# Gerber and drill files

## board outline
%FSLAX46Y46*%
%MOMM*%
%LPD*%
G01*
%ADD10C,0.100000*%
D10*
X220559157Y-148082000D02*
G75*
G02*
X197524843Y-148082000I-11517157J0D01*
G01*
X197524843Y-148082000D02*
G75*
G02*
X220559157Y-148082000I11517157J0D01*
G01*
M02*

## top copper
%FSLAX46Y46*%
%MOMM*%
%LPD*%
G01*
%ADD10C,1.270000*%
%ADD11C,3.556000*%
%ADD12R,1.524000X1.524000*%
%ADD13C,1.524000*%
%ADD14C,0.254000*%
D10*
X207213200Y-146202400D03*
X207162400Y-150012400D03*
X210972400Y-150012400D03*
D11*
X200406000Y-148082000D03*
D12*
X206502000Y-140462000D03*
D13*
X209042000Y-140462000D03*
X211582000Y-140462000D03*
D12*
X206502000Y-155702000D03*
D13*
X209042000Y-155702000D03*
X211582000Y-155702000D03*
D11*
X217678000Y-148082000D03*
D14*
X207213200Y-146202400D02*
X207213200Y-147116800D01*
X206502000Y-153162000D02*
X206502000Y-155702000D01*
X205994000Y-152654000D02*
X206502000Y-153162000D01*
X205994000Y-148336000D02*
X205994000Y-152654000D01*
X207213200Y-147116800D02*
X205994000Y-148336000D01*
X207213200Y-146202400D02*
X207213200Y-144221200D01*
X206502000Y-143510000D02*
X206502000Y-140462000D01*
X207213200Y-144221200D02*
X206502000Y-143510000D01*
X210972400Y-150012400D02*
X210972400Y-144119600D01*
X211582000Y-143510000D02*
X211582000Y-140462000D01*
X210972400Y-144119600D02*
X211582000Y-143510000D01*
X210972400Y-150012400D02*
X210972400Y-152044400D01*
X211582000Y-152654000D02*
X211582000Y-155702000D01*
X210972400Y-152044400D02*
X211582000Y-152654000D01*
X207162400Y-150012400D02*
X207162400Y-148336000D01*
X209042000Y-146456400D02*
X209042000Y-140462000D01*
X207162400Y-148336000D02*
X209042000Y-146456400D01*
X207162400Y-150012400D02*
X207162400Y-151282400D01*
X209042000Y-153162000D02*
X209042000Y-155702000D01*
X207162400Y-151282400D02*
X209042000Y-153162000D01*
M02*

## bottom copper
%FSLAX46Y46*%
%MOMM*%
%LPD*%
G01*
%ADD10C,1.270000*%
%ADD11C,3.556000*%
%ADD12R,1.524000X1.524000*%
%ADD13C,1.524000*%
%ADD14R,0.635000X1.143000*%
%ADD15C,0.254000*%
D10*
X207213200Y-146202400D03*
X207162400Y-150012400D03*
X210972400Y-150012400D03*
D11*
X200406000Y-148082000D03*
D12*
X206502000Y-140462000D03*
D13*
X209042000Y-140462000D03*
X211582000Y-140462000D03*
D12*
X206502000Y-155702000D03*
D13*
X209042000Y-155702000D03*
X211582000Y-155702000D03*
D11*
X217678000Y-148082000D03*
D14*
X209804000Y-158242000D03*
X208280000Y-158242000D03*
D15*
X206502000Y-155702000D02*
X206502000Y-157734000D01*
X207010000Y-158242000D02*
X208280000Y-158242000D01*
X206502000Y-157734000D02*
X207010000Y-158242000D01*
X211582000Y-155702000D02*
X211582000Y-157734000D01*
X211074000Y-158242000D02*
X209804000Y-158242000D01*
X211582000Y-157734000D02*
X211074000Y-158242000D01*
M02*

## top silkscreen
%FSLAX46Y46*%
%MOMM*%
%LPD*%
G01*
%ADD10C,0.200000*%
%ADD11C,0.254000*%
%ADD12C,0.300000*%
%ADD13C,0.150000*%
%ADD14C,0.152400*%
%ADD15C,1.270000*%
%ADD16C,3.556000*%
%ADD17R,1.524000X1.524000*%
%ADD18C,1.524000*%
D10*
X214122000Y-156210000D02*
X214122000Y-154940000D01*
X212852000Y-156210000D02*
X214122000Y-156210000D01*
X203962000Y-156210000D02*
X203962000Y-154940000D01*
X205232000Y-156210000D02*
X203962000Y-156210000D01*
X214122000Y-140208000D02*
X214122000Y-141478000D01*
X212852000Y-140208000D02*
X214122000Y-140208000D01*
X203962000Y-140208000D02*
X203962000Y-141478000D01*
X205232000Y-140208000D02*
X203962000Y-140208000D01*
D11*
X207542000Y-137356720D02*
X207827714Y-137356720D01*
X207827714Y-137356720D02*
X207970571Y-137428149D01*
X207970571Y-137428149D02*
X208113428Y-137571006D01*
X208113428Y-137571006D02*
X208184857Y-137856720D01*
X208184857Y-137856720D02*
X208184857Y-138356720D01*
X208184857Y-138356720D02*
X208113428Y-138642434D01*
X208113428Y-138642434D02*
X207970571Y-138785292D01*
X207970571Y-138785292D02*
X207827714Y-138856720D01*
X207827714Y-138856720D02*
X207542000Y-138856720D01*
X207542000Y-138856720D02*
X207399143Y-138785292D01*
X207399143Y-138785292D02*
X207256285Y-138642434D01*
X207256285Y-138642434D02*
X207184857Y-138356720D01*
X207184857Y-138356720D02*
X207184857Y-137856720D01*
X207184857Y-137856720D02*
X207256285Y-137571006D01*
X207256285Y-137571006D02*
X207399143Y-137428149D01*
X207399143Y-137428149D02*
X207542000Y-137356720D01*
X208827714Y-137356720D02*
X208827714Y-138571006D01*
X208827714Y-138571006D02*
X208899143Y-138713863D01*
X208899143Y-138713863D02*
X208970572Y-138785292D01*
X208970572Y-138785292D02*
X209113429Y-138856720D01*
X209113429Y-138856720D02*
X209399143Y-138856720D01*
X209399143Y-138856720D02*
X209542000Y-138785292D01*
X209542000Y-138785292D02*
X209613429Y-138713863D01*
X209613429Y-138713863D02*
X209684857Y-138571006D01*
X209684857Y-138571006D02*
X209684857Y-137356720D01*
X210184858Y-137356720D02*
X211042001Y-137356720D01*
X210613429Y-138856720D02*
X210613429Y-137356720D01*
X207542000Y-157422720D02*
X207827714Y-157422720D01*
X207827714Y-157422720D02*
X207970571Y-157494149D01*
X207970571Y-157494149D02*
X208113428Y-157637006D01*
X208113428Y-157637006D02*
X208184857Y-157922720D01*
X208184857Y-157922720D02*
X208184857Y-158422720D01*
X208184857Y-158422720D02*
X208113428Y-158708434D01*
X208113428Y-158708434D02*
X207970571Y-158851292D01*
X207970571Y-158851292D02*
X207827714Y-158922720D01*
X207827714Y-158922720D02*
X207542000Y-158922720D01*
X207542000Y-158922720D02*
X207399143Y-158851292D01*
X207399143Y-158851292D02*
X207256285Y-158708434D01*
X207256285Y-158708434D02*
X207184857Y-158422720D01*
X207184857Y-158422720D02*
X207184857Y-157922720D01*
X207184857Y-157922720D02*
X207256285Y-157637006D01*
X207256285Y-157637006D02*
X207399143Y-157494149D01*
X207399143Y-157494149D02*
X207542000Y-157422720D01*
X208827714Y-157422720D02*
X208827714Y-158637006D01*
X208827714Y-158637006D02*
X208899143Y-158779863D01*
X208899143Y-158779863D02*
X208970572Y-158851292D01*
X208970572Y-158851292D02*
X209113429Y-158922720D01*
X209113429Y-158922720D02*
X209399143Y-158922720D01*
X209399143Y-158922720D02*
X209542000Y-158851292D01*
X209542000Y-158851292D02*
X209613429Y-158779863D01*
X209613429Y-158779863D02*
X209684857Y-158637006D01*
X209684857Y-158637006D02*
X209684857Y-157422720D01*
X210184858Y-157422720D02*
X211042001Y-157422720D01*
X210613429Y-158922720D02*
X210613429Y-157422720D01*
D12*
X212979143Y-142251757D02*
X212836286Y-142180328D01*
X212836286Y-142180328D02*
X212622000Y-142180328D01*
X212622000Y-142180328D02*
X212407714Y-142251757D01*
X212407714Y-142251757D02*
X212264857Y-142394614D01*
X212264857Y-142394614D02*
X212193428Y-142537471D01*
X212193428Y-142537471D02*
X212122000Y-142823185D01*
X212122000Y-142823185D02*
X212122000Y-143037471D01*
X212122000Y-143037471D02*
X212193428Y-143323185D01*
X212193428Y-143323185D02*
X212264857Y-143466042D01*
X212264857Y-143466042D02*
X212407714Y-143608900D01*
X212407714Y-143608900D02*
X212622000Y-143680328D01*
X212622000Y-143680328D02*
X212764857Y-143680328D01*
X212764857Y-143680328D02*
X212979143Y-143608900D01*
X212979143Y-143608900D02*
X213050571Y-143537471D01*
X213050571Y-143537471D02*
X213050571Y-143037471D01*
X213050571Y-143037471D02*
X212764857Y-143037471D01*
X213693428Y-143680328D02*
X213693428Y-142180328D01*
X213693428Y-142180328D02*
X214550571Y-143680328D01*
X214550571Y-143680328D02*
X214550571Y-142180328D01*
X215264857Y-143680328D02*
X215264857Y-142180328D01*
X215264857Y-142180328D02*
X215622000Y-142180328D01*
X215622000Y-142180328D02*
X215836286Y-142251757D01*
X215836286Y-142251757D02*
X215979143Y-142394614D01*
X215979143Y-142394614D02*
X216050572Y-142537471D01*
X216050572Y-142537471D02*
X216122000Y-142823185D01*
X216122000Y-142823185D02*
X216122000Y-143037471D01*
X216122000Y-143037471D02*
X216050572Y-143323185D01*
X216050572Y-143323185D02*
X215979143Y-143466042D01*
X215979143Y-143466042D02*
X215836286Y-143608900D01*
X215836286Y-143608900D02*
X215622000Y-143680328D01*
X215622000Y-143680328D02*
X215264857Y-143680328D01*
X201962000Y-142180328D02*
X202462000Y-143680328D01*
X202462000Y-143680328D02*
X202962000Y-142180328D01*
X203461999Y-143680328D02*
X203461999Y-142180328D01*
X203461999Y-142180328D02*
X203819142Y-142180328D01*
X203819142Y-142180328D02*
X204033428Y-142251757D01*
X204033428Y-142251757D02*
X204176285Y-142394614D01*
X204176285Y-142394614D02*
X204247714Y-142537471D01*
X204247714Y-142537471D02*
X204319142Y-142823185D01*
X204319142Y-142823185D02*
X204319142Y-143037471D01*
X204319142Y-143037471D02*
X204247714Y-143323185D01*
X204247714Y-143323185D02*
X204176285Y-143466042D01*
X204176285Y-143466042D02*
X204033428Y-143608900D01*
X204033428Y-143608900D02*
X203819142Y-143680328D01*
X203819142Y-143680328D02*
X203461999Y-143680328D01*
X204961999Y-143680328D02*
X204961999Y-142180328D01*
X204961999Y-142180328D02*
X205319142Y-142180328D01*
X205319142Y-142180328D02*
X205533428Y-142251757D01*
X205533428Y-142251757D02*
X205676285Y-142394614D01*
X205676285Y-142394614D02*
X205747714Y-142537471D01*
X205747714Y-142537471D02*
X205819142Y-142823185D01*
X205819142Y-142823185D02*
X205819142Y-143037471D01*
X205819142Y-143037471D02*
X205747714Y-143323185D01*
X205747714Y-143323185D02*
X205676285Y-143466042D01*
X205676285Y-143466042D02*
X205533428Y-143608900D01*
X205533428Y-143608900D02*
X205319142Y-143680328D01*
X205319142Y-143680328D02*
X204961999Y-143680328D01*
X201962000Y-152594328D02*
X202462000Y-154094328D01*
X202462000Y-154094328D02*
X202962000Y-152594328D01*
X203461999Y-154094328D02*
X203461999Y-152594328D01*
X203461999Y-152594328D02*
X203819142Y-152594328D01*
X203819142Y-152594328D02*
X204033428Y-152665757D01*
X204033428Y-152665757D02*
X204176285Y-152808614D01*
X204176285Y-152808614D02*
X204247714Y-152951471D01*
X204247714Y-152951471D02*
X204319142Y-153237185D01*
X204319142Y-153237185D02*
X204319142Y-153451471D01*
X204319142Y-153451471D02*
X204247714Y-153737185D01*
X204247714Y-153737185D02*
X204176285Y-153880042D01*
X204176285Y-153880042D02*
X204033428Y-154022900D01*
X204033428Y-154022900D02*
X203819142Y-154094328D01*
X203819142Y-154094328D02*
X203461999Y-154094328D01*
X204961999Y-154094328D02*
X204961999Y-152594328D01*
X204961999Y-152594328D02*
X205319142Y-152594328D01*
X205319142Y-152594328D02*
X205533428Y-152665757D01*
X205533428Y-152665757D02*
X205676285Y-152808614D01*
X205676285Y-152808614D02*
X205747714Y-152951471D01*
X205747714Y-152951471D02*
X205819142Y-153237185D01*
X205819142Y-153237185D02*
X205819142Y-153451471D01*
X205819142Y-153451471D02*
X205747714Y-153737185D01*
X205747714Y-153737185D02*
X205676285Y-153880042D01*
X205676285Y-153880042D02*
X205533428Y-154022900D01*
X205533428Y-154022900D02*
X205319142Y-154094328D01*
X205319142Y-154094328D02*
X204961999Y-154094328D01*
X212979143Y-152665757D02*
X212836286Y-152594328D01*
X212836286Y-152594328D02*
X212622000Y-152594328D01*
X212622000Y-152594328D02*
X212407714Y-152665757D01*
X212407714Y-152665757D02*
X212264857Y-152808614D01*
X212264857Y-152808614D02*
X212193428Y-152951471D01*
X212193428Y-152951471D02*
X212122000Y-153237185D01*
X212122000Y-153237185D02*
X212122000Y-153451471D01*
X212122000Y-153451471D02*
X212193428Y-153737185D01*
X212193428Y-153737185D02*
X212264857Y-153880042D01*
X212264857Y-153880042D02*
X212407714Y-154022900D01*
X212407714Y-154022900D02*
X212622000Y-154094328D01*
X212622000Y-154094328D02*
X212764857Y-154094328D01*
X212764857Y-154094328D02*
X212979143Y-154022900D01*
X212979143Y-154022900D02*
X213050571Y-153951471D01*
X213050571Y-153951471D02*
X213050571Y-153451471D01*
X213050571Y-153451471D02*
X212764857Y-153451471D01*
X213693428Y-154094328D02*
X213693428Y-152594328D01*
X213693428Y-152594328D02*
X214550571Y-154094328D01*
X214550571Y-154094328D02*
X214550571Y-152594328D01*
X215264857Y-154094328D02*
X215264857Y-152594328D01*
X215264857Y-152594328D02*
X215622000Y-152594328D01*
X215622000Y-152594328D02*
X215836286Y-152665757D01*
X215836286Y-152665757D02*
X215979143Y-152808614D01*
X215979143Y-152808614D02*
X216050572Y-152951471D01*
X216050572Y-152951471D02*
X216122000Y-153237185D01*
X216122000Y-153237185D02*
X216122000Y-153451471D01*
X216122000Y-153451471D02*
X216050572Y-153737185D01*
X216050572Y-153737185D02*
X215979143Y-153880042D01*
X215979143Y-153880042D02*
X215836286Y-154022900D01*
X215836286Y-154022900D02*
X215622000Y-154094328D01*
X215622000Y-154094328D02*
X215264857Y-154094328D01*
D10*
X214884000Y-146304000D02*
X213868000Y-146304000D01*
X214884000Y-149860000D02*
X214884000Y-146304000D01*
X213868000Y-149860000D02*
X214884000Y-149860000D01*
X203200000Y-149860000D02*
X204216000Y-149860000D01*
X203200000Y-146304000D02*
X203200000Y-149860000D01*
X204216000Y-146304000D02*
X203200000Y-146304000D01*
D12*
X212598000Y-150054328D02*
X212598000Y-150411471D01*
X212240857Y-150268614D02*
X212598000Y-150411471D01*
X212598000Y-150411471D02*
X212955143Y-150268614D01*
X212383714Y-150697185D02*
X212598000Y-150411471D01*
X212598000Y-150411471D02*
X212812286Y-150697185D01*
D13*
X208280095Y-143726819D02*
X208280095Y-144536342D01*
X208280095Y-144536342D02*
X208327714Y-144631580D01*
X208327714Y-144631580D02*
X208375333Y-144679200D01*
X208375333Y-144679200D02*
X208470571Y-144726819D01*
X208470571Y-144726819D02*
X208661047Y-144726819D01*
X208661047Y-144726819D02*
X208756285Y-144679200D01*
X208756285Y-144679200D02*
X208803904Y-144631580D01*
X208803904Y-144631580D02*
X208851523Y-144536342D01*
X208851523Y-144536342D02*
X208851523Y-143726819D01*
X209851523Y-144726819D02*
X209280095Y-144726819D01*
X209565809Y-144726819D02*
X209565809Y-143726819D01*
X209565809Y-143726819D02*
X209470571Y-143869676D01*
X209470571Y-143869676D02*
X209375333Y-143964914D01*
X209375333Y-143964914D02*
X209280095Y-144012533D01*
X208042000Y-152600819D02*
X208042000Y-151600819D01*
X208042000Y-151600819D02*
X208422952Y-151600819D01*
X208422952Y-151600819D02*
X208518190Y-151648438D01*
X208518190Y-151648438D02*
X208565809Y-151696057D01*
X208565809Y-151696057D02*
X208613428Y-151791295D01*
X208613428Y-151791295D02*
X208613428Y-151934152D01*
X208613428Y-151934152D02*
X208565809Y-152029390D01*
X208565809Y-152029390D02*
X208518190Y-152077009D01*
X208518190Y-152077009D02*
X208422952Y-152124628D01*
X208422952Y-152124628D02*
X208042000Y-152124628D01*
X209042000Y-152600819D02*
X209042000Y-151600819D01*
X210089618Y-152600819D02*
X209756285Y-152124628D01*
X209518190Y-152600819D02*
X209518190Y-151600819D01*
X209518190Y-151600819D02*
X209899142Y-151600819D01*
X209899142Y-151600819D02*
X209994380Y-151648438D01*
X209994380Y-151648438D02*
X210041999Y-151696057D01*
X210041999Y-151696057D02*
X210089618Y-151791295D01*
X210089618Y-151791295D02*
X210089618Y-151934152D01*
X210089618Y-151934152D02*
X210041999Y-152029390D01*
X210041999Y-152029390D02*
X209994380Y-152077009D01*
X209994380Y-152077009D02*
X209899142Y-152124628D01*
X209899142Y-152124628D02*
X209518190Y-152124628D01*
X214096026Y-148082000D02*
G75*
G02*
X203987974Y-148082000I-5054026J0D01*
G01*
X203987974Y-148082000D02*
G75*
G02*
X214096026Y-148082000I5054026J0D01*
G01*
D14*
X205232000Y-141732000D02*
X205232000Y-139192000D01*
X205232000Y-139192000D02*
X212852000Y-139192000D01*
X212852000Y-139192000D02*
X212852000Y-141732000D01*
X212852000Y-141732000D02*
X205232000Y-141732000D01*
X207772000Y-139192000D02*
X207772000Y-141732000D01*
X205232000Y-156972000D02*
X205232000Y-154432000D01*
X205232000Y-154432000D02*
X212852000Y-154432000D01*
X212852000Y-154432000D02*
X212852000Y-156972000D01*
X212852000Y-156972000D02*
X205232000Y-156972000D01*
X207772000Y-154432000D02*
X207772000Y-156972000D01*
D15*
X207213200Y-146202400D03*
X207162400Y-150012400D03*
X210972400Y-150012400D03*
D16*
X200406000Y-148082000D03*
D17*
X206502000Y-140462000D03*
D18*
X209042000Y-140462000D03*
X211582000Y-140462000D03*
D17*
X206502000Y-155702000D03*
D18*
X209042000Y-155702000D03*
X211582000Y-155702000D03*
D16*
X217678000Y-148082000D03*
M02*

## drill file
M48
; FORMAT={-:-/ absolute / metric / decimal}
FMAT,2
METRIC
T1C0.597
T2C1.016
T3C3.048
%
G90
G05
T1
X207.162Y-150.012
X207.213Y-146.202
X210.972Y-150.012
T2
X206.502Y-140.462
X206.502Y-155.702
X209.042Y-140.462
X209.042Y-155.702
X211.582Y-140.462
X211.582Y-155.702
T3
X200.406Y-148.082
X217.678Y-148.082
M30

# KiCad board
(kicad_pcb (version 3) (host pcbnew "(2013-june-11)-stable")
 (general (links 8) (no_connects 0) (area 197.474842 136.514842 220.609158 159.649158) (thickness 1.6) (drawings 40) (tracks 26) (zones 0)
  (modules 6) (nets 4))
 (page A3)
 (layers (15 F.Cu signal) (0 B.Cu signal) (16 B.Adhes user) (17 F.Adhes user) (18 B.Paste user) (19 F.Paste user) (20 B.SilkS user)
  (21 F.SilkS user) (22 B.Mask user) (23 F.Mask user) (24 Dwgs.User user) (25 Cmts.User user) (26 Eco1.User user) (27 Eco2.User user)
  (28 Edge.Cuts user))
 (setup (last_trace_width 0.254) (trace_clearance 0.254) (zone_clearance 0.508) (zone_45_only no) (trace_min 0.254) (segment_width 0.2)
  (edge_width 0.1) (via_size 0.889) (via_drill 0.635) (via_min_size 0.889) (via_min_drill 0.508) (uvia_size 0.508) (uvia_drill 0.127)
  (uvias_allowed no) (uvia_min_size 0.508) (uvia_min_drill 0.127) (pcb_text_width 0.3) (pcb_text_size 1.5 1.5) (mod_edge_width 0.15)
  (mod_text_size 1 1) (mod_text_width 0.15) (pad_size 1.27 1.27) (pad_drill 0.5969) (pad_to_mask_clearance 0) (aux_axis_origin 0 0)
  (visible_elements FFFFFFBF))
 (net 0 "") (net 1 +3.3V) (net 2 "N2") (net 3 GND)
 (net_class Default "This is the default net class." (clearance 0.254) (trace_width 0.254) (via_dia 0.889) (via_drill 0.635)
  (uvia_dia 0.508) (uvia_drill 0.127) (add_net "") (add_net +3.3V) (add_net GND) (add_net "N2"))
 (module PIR (layer F.Cu) (at 209.042 148.082)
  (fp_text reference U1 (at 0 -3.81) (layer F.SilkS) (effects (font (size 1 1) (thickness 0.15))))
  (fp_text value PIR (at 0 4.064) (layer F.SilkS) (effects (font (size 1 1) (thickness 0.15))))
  (fp_circle (center 0 0) (end -3.9116 3.2004) (layer F.SilkS) (width 0.15))
  (pad 1 thru_hole circle (at -1.8288 -1.8796 180) (size 1.27 1.27) (drill 0.5969) (layers *.Cu *.Mask F.SilkS) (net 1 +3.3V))
  (pad 2 thru_hole circle (at -1.8796 1.9304 180) (size 1.27 1.27) (drill 0.5969) (layers *.Cu *.Mask F.SilkS) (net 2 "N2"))
  (pad 3 thru_hole circle (at 1.9304 1.9304 180) (size 1.27 1.27) (drill 0.5969) (layers *.Cu *.Mask F.SilkS) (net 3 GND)))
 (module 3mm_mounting (layer F.Cu) (at 200.406 148.082)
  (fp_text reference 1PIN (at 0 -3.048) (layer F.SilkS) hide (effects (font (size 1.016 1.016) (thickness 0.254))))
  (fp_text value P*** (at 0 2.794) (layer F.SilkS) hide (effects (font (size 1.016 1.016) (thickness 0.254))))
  (pad "" thru_hole circle (at 0 0) (size 3.556 3.556) (drill 3.048) (layers *.Cu *.Mask F.SilkS)))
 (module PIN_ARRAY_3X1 (layer F.Cu) (at 209.042 140.462)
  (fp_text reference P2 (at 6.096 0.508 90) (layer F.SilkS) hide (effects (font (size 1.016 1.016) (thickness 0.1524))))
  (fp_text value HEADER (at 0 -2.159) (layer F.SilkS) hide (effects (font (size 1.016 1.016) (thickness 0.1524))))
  (fp_line (start -3.81 1.27) (end -3.81 -1.27) (layer F.SilkS) (width 0.1524))
  (fp_line (start -3.81 -1.27) (end 3.81 -1.27) (layer F.SilkS) (width 0.1524))
  (fp_line (start 3.81 -1.27) (end 3.81 1.27) (layer F.SilkS) (width 0.1524))
  (fp_line (start 3.81 1.27) (end -3.81 1.27) (layer F.SilkS) (width 0.1524))
  (fp_line (start -1.27 -1.27) (end -1.27 1.27) (layer F.SilkS) (width 0.1524))
  (pad 1 thru_hole rect (at -2.54 0) (size 1.524 1.524) (drill 1.016) (layers *.Cu *.Mask F.SilkS) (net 1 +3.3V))
  (pad 2 thru_hole circle (at 0 0) (size 1.524 1.524) (drill 1.016) (layers *.Cu *.Mask F.SilkS) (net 2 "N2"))
  (pad 3 thru_hole circle (at 2.54 0) (size 1.524 1.524) (drill 1.016) (layers *.Cu *.Mask F.SilkS) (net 3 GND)))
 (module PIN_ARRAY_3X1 (layer F.Cu) (at 209.042 155.702)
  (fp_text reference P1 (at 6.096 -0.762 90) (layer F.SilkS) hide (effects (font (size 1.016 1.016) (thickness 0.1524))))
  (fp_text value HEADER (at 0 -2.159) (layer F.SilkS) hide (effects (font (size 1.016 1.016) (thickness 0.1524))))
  (fp_line (start -3.81 1.27) (end -3.81 -1.27) (layer F.SilkS) (width 0.1524))
  (fp_line (start -3.81 -1.27) (end 3.81 -1.27) (layer F.SilkS) (width 0.1524))
  (fp_line (start 3.81 -1.27) (end 3.81 1.27) (layer F.SilkS) (width 0.1524))
  (fp_line (start 3.81 1.27) (end -3.81 1.27) (layer F.SilkS) (width 0.1524))
  (fp_line (start -1.27 -1.27) (end -1.27 1.27) (layer F.SilkS) (width 0.1524))
  (pad 1 thru_hole rect (at -2.54 0) (size 1.524 1.524) (drill 1.016) (layers *.Cu *.Mask F.SilkS) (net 1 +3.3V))
  (pad 2 thru_hole circle (at 0 0) (size 1.524 1.524) (drill 1.016) (layers *.Cu *.Mask F.SilkS) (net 2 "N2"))
  (pad 3 thru_hole circle (at 2.54 0) (size 1.524 1.524) (drill 1.016) (layers *.Cu *.Mask F.SilkS) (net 3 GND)))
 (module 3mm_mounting (layer F.Cu) (at 217.678 148.082)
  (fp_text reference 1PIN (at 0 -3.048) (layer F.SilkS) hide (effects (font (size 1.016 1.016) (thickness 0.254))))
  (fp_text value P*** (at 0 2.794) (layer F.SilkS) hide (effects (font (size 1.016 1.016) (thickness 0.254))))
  (pad "" thru_hole circle (at 0 0) (size 3.556 3.556) (drill 3.048) (layers *.Cu *.Mask F.SilkS)))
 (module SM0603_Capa (layer B.Cu) (at 209.042 158.242 180)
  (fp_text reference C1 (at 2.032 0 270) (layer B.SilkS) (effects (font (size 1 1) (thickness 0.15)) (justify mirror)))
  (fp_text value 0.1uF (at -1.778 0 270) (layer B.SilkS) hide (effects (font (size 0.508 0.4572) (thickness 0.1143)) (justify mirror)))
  (pad 1 smd rect (at -0.762 0 180) (size 0.635 1.143) (layers B.Cu B.Paste B.Mask) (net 3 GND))
  (pad 2 smd rect (at 0.762 0 180) (size 0.635 1.143) (layers B.Cu B.Paste B.Mask) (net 1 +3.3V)))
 (gr_line (start 214.122 156.21) (end 214.122 154.94) (angle 90) (layer F.SilkS) (width 0.2))
 (gr_line (start 212.852 156.21) (end 214.122 156.21) (angle 90) (layer F.SilkS) (width 0.2))
 (gr_line (start 203.962 156.21) (end 203.962 154.94) (angle 90) (layer F.SilkS) (width 0.2))
 (gr_line (start 205.232 156.21) (end 203.962 156.21) (angle 90) (layer F.SilkS) (width 0.2))
 (gr_line (start 214.122 140.208) (end 214.122 141.478) (angle 90) (layer F.SilkS) (width 0.2))
 (gr_line (start 212.852 140.208) (end 214.122 140.208) (angle 90) (layer F.SilkS) (width 0.2))
 (gr_line (start 203.962 140.208) (end 203.962 141.478) (angle 90) (layer F.SilkS) (width 0.2))
 (gr_line (start 205.232 140.208) (end 203.962 140.208) (angle 90) (layer F.SilkS) (width 0.2))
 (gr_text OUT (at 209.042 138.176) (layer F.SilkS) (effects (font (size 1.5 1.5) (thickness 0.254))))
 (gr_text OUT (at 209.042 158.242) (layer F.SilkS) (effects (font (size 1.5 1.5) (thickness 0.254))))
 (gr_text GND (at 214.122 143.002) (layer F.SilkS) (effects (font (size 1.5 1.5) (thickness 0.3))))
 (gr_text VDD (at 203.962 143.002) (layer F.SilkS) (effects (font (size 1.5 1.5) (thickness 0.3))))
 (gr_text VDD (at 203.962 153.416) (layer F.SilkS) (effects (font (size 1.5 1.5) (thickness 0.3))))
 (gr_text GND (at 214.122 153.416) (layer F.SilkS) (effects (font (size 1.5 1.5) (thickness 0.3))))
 (gr_line (start 214.884 146.304) (end 213.868 146.304) (angle 90) (layer F.SilkS) (width 0.2))
 (gr_line (start 214.884 149.86) (end 214.884 146.304) (angle 90) (layer F.SilkS) (width 0.2))
 (gr_line (start 213.868 149.86) (end 214.884 149.86) (angle 90) (layer F.SilkS) (width 0.2))
 (gr_line (start 203.2 149.86) (end 204.216 149.86) (angle 90) (layer F.SilkS) (width 0.2))
 (gr_line (start 203.2 146.304) (end 203.2 149.86) (angle 90) (layer F.SilkS) (width 0.2))
 (gr_line (start 204.216 146.304) (end 203.2 146.304) (angle 90) (layer F.SilkS) (width 0.2))
 (gr_circle (center 209.042 148.082) (end 216.662 156.718) (layer Edge.Cuts) (width 0.1))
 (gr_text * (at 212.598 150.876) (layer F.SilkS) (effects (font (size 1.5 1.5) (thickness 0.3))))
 (segment (start 206.502 155.702) (end 206.502 157.734) (width 0.254) (layer B.Cu) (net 1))
 (segment (start 207.01 158.242) (end 208.28 158.242) (width 0.254) (layer B.Cu) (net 1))
 (segment (start 206.502 157.734) (end 207.01 158.242) (width 0.254) (layer B.Cu) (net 1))
 (segment (start 207.2132 146.2024) (end 207.2132 147.1168) (width 0.254) (layer F.Cu) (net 1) (status 10))
 (segment (start 206.502 153.162) (end 206.502 155.702) (width 0.254) (layer F.Cu) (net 1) (status 20))
 (segment (start 205.994 152.654) (end 206.502 153.162) (width 0.254) (layer F.Cu) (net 1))
 (segment (start 205.994 148.336) (end 205.994 152.654) (width 0.254) (layer F.Cu) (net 1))
 (segment (start 207.2132 147.1168) (end 205.994 148.336) (width 0.254) (layer F.Cu) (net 1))
 (segment (start 207.2132 146.2024) (end 207.2132 144.2212) (width 0.254) (layer F.Cu) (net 1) (status 10))
 (segment (start 206.502 143.51) (end 206.502 140.462) (width 0.254) (layer F.Cu) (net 1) (status 20))
 (segment (start 207.2132 144.2212) (end 206.502 143.51) (width 0.254) (layer F.Cu) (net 1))
 (segment (start 211.582 155.702) (end 211.582 157.734) (width 0.254) (layer B.Cu) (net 3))
 (segment (start 211.074 158.242) (end 209.804 158.242) (width 0.254) (layer B.Cu) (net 3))
 (segment (start 211.582 157.734) (end 211.074 158.242) (width 0.254) (layer B.Cu) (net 3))
 (segment (start 210.9724 150.0124) (end 210.9724 144.1196) (width 0.254) (layer F.Cu) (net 3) (status 10))
 (segment (start 211.582 143.51) (end 211.582 140.462) (width 0.254) (layer F.Cu) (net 3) (status 20))
 (segment (start 210.9724 144.1196) (end 211.582 143.51) (width 0.254) (layer F.Cu) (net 3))
 (segment (start 210.9724 150.0124) (end 210.9724 152.0444) (width 0.254) (layer F.Cu) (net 3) (status 10))
 (segment (start 211.582 152.654) (end 211.582 155.702) (width 0.254) (layer F.Cu) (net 3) (status 20))
 (segment (start 210.9724 152.0444) (end 211.582 152.654) (width 0.254) (layer F.Cu) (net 3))
 (segment (start 207.1624 150.0124) (end 207.1624 148.336) (width 0.254) (layer F.Cu) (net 2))
 (segment (start 209.042 146.4564) (end 209.042 140.462) (width 0.254) (layer F.Cu) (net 2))
 (segment (start 207.1624 148.336) (end 209.042 146.4564) (width 0.254) (layer F.Cu) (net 2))
 (segment (start 207.1624 150.0124) (end 207.1624 151.2824) (width 0.254) (layer F.Cu) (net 2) (status 10))
 (segment (start 209.042 153.162) (end 209.042 155.702) (width 0.254) (layer F.Cu) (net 2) (status 20))
 (segment (start 207.1624 151.2824) (end 209.042 153.162) (width 0.254) (layer F.Cu) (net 2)))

